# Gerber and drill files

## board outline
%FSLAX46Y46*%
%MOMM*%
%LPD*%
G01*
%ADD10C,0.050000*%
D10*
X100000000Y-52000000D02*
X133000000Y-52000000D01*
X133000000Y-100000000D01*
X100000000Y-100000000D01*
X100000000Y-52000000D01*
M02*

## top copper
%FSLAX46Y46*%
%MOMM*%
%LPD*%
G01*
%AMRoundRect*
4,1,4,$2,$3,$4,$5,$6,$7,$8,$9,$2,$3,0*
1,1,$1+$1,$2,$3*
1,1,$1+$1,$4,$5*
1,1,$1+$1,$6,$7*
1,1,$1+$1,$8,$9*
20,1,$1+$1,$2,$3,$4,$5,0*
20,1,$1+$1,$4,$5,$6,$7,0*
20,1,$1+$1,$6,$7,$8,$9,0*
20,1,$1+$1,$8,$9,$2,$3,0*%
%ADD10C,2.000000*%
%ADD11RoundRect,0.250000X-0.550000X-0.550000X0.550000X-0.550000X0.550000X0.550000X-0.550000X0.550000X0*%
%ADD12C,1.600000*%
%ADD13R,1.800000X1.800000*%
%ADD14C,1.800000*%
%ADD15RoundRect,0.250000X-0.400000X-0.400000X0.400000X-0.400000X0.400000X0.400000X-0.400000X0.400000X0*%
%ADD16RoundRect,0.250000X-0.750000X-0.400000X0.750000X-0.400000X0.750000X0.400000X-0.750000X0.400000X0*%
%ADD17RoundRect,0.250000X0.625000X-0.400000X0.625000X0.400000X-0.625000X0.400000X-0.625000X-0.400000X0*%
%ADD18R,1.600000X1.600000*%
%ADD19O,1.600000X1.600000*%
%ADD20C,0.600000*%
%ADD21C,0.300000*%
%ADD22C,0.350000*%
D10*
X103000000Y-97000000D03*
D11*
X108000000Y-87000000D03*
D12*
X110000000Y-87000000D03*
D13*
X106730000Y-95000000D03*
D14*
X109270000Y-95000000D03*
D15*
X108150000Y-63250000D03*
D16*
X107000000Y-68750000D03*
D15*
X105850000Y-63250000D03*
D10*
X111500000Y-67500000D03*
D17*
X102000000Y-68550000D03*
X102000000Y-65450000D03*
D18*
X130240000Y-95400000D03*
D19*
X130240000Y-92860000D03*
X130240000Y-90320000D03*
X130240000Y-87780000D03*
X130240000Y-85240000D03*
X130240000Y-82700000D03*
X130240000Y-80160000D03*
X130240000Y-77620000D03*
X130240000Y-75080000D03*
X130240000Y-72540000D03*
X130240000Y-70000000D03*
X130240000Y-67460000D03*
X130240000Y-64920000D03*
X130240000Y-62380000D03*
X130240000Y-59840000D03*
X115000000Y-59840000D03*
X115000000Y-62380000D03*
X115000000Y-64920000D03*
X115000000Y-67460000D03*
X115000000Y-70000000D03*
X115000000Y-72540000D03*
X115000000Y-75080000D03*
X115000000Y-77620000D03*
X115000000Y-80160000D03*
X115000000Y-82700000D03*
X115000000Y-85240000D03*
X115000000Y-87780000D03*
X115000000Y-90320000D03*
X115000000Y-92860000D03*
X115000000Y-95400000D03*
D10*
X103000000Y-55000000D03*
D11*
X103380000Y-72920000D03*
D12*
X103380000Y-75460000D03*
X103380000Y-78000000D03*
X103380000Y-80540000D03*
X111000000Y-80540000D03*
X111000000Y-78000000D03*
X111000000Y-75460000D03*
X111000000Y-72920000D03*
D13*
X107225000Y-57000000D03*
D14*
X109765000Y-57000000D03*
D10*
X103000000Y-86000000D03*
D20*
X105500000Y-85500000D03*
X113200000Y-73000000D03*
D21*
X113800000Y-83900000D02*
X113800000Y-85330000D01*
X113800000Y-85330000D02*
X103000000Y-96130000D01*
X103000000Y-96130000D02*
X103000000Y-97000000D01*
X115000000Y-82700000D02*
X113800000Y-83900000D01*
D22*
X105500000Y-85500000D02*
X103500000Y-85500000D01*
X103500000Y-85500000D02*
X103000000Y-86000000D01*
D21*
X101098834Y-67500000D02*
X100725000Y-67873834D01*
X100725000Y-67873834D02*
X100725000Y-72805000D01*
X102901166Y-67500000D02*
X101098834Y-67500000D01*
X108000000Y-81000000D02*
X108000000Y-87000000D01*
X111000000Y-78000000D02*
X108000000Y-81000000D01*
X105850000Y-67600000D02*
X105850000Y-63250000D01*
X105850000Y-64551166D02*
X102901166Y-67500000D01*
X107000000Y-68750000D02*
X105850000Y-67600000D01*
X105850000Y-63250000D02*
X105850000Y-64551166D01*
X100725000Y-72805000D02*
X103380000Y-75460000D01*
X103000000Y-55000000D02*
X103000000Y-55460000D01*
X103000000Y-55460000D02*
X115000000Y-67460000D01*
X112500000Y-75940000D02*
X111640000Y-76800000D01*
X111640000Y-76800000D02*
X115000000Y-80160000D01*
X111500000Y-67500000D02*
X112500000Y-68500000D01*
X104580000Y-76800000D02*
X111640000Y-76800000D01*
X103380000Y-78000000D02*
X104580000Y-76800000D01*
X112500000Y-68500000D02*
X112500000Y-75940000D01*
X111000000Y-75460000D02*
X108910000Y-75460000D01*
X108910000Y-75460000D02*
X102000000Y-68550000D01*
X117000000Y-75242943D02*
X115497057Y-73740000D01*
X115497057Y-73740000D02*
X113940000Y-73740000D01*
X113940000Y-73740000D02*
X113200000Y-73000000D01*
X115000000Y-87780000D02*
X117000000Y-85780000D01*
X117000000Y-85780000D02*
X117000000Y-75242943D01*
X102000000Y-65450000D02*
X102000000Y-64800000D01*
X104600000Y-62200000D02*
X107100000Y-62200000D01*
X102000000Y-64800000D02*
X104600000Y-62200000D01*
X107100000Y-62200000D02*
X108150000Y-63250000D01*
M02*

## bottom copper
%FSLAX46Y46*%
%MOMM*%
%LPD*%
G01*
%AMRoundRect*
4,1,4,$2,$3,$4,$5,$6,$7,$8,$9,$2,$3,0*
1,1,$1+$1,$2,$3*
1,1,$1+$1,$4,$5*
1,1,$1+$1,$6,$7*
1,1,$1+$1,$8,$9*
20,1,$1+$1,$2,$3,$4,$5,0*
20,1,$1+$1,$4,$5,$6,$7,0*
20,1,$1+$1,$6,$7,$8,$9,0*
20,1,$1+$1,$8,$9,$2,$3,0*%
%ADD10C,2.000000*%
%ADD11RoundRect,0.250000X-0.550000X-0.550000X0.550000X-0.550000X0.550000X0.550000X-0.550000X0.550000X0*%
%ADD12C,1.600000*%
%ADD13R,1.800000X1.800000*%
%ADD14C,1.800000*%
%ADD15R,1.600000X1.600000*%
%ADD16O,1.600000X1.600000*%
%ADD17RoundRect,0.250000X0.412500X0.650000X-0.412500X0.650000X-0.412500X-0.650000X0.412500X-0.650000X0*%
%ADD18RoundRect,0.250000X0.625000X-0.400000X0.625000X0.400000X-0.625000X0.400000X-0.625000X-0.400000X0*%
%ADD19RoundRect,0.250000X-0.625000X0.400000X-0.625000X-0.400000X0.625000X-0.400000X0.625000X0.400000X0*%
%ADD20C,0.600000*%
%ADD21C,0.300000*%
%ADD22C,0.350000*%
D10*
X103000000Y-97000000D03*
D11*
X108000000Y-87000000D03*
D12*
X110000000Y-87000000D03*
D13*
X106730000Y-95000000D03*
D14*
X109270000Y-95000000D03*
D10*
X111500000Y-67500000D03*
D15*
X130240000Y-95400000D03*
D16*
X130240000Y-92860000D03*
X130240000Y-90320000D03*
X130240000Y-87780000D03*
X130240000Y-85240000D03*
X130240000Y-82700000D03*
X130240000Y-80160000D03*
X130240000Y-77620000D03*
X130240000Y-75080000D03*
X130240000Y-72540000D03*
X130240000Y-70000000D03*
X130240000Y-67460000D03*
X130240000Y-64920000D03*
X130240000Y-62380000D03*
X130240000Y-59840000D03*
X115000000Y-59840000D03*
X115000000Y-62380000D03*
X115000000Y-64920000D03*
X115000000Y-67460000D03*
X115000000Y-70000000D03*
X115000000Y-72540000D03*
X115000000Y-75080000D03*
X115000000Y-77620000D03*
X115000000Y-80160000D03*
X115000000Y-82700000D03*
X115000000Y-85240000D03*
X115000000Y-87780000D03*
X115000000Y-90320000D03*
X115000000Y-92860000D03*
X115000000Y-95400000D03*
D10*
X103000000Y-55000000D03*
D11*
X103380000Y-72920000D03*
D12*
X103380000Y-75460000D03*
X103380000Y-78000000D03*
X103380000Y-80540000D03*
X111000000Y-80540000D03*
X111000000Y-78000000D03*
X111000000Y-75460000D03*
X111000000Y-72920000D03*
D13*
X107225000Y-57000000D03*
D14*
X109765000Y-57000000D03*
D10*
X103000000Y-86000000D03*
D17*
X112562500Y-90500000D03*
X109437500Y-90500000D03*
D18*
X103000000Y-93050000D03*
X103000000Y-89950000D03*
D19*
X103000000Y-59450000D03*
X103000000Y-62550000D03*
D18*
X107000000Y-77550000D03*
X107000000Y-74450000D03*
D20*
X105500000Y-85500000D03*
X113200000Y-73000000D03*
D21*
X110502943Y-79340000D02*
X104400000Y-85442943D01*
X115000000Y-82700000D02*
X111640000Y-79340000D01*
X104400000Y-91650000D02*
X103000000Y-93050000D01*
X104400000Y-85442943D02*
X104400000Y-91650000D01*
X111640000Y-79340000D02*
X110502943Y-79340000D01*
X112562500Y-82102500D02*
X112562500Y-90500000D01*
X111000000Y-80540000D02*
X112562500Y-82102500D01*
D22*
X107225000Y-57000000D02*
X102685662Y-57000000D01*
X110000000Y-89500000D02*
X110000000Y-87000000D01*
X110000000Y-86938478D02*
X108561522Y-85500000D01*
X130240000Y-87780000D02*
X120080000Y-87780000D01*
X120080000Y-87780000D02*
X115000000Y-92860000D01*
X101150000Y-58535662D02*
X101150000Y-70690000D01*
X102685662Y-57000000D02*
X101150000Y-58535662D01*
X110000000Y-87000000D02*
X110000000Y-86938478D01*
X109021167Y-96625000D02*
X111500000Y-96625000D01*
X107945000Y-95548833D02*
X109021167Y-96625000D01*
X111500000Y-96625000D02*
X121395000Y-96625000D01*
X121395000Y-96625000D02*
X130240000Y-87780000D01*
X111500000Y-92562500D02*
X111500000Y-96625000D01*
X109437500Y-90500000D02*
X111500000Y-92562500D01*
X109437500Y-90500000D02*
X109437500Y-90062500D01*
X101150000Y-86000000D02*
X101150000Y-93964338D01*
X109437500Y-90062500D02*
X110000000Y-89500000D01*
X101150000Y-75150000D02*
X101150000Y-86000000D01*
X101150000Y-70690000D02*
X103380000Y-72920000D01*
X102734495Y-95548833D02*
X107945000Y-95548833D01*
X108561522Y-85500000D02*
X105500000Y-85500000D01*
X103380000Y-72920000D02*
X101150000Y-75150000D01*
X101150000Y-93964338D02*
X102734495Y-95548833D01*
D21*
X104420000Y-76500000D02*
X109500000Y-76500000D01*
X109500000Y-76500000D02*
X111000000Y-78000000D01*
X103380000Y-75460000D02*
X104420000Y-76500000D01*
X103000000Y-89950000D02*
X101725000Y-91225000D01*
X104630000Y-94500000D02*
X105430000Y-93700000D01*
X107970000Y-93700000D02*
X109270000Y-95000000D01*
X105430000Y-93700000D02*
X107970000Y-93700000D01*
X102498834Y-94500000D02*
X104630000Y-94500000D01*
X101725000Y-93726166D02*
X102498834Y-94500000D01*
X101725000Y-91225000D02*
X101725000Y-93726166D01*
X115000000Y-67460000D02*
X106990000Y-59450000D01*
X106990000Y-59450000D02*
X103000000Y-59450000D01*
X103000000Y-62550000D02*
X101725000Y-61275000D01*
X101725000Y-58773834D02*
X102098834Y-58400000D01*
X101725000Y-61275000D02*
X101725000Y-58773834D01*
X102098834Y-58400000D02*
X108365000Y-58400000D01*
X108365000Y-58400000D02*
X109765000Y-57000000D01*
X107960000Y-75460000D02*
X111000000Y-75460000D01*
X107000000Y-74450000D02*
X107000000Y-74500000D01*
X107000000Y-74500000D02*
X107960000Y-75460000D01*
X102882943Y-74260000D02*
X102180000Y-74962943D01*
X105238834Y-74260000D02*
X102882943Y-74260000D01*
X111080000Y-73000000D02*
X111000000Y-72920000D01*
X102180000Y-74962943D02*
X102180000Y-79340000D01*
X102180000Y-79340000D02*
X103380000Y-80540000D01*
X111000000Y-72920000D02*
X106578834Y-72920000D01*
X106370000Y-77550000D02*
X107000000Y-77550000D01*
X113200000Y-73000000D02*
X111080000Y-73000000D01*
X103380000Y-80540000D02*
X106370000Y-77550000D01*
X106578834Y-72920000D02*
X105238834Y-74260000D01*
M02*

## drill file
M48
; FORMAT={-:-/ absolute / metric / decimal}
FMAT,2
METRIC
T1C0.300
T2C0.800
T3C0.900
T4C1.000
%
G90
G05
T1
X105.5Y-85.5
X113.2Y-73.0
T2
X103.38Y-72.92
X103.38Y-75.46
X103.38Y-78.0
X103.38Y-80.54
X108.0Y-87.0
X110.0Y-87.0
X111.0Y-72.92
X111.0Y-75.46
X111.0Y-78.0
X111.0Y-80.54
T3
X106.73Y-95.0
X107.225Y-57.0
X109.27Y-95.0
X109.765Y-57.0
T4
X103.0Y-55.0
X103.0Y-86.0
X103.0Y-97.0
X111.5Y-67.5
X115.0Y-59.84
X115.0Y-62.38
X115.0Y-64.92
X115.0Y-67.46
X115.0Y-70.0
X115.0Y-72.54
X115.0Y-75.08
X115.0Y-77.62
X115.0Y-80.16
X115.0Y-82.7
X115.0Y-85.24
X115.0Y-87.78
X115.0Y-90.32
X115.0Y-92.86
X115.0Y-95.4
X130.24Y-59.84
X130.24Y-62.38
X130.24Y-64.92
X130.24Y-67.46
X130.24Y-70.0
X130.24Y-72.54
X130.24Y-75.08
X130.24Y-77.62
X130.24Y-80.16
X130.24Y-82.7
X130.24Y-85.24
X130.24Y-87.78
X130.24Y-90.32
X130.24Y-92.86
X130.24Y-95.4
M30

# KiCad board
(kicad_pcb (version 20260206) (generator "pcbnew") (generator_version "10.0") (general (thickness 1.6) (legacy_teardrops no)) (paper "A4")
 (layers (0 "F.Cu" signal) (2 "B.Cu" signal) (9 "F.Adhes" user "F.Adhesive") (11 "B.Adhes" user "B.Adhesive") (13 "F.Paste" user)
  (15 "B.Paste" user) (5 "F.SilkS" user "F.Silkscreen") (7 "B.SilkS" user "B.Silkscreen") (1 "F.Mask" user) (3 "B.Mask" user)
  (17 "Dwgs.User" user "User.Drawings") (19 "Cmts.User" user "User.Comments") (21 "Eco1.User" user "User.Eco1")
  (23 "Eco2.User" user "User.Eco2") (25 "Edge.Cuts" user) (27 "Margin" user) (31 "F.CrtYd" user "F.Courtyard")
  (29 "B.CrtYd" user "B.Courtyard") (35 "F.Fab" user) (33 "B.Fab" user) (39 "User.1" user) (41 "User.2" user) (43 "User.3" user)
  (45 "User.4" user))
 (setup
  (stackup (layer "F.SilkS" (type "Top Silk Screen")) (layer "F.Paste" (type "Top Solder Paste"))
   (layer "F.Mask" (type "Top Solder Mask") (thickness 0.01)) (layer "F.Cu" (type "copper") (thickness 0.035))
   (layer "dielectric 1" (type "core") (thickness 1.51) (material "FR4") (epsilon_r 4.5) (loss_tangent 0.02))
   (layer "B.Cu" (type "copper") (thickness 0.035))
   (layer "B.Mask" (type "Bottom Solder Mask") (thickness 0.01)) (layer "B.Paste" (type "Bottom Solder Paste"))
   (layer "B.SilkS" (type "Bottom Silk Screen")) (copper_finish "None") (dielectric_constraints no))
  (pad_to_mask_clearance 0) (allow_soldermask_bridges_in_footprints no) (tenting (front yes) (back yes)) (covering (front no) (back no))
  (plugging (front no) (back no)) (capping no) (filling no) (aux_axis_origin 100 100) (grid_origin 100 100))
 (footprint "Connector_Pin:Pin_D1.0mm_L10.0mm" (layer "F.Cu") (at 103 97)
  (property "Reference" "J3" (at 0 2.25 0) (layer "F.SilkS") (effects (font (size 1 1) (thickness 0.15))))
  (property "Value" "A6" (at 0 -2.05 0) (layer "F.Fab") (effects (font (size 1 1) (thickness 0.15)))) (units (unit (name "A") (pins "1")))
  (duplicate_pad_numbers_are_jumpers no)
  (pad "1" thru_hole circle (at 0 0) (size 2 2) (drill 1) (layers "*.Cu" "*.Mask") (remove_unused_layers no) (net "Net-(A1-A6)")))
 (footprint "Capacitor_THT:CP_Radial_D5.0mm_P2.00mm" (layer "F.Cu") (at 108 87)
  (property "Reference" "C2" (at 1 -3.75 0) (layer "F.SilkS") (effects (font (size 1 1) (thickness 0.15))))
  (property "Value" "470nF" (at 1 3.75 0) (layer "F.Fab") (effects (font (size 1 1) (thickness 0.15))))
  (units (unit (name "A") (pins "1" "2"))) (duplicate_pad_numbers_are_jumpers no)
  (pad "1" thru_hole roundrect (at 0 0) (size 1.6 1.6) (drill 0.8) (layers "*.Cu" "*.Mask") (remove_unused_layers no)
   (roundrect_rratio 0.15625) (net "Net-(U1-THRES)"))
  (pad "2" thru_hole circle (at 2 0) (size 1.6 1.6) (drill 0.8) (layers "*.Cu" "*.Mask") (remove_unused_layers no) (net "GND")))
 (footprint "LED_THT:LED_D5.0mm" (layer "F.Cu") (at 106.73 95)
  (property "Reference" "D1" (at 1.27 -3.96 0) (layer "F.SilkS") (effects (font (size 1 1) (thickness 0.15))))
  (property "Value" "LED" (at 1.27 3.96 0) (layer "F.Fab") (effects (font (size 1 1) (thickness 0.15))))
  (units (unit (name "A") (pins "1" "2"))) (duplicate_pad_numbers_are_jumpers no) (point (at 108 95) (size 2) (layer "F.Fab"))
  (pad "1" thru_hole rect (at 0 0) (size 1.8 1.8) (drill 0.9) (layers "*.Cu" "*.Mask") (remove_unused_layers no) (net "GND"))
  (pad "2" thru_hole circle (at 2.54 0) (size 1.8 1.8) (drill 0.9) (layers "*.Cu" "*.Mask") (remove_unused_layers no) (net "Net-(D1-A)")))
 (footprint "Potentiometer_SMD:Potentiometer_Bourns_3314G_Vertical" (layer "F.Cu") (at 107 66)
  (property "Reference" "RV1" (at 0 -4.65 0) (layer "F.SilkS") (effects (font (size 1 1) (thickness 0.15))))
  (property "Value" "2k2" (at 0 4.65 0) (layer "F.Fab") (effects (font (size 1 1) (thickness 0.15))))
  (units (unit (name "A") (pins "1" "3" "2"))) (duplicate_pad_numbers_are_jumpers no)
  (pad "1" smd roundrect (at 1.15 -2.75) (size 1.3 1.3) (layers "F.Cu" "F.Mask" "F.Paste") (roundrect_rratio 0.192308) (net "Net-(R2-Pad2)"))
  (pad "2" smd roundrect (at 0 2.75) (size 2 1.3) (layers "F.Cu" "F.Mask" "F.Paste") (roundrect_rratio 0.192308) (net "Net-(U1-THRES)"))
  (pad "3" smd roundrect (at -1.15 -2.75) (size 1.3 1.3) (layers "F.Cu" "F.Mask" "F.Paste") (roundrect_rratio 0.192308)
   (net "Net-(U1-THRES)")))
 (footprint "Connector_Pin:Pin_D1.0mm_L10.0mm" (layer "F.Cu") (at 111.5 67.5)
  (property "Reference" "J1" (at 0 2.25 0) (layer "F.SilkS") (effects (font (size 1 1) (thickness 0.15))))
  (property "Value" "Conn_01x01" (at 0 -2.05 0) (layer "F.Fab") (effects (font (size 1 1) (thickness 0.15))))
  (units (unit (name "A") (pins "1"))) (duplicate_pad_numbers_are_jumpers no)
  (pad "1" thru_hole circle (at 0 0) (size 2 2) (drill 1) (layers "*.Cu" "*.Mask") (remove_unused_layers no) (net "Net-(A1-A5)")))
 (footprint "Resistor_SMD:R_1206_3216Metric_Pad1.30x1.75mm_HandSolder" (layer "F.Cu") (at 102 67 90)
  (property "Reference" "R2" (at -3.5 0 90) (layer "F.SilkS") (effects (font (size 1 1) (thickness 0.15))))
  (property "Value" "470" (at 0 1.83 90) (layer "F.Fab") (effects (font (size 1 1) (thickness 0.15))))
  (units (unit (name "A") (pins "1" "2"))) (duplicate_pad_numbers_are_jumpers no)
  (pad "1" smd roundrect (at -1.55 0 90) (size 1.3 1.75) (layers "F.Cu" "F.Mask" "F.Paste") (roundrect_rratio 0.192308)
   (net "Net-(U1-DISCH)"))
  (pad "2" smd roundrect (at 1.55 0 90) (size 1.3 1.75) (layers "F.Cu" "F.Mask" "F.Paste") (roundrect_rratio 0.192308) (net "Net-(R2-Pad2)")))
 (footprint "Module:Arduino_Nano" (layer "F.Cu") (at 130.24 95.4 180)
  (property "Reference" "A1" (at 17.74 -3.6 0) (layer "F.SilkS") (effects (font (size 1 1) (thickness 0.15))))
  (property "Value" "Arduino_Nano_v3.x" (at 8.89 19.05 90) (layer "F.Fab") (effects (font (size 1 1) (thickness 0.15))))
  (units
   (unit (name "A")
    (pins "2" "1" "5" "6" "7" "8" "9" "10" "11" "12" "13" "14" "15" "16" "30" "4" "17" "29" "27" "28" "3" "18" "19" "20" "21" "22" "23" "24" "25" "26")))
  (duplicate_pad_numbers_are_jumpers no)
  (pad "1" thru_hole rect (at 0 0 180) (size 1.6 1.6) (drill 1) (layers "*.Cu" "*.Mask") (remove_unused_layers no)
   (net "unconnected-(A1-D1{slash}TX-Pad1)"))
  (pad "2" thru_hole oval (at 0 2.54 180) (size 1.6 1.6) (drill 1) (layers "*.Cu" "*.Mask") (remove_unused_layers no)
   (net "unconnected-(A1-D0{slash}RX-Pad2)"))
  (pad "3" thru_hole oval (at 0 5.08 180) (size 1.6 1.6) (drill 1) (layers "*.Cu" "*.Mask") (remove_unused_layers no)
   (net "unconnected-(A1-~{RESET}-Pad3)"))
  (pad "4" thru_hole oval (at 0 7.62 180) (size 1.6 1.6) (drill 1) (layers "*.Cu" "*.Mask") (remove_unused_layers no) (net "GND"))
  (pad "5" thru_hole oval (at 0 10.16 180) (size 1.6 1.6) (drill 1) (layers "*.Cu" "*.Mask") (remove_unused_layers no)
   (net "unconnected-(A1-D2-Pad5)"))
  (pad "6" thru_hole oval (at 0 12.7 180) (size 1.6 1.6) (drill 1) (layers "*.Cu" "*.Mask") (remove_unused_layers no)
   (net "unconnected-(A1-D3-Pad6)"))
  (pad "7" thru_hole oval (at 0 15.24 180) (size 1.6 1.6) (drill 1) (layers "*.Cu" "*.Mask") (remove_unused_layers no)
   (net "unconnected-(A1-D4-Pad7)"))
  (pad "8" thru_hole oval (at 0 17.78 180) (size 1.6 1.6) (drill 1) (layers "*.Cu" "*.Mask") (remove_unused_layers no)
   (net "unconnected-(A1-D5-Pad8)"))
  (pad "9" thru_hole oval (at 0 20.32 180) (size 1.6 1.6) (drill 1) (layers "*.Cu" "*.Mask") (remove_unused_layers no)
   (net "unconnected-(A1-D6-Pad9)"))
  (pad "10" thru_hole oval (at 0 22.86 180) (size 1.6 1.6) (drill 1) (layers "*.Cu" "*.Mask") (remove_unused_layers no)
   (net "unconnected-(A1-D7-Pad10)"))
  (pad "11" thru_hole oval (at 0 25.4 180) (size 1.6 1.6) (drill 1) (layers "*.Cu" "*.Mask") (remove_unused_layers no)
   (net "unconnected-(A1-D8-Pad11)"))
  (pad "12" thru_hole oval (at 0 27.94 180) (size 1.6 1.6) (drill 1) (layers "*.Cu" "*.Mask") (remove_unused_layers no)
   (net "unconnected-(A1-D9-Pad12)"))
  (pad "13" thru_hole oval (at 0 30.48 180) (size 1.6 1.6) (drill 1) (layers "*.Cu" "*.Mask") (remove_unused_layers no)
   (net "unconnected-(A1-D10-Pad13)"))
  (pad "14" thru_hole oval (at 0 33.02 180) (size 1.6 1.6) (drill 1) (layers "*.Cu" "*.Mask") (remove_unused_layers no)
   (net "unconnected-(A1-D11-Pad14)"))
  (pad "15" thru_hole oval (at 0 35.56 180) (size 1.6 1.6) (drill 1) (layers "*.Cu" "*.Mask") (remove_unused_layers no)
   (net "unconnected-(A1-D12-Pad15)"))
  (pad "16" thru_hole oval (at 15.24 35.56 180) (size 1.6 1.6) (drill 1) (layers "*.Cu" "*.Mask") (remove_unused_layers no)
   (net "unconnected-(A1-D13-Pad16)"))
  (pad "17" thru_hole oval (at 15.24 33.02 180) (size 1.6 1.6) (drill 1) (layers "*.Cu" "*.Mask") (remove_unused_layers no)
   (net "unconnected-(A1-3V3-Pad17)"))
  (pad "18" thru_hole oval (at 15.24 30.48 180) (size 1.6 1.6) (drill 1) (layers "*.Cu" "*.Mask") (remove_unused_layers no)
   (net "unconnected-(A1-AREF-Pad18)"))
  (pad "19" thru_hole oval (at 15.24 27.94 180) (size 1.6 1.6) (drill 1) (layers "*.Cu" "*.Mask") (remove_unused_layers no)
   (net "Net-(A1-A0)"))
  (pad "20" thru_hole oval (at 15.24 25.4 180) (size 1.6 1.6) (drill 1) (layers "*.Cu" "*.Mask") (remove_unused_layers no)
   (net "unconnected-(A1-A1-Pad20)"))
  (pad "21" thru_hole oval (at 15.24 22.86 180) (size 1.6 1.6) (drill 1) (layers "*.Cu" "*.Mask") (remove_unused_layers no)
   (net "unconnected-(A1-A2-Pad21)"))
  (pad "22" thru_hole oval (at 15.24 20.32 180) (size 1.6 1.6) (drill 1) (layers "*.Cu" "*.Mask") (remove_unused_layers no)
   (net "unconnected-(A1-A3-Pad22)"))
  (pad "23" thru_hole oval (at 15.24 17.78 180) (size 1.6 1.6) (drill 1) (layers "*.Cu" "*.Mask") (remove_unused_layers no)
   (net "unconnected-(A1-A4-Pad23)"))
  (pad "24" thru_hole oval (at 15.24 15.24 180) (size 1.6 1.6) (drill 1) (layers "*.Cu" "*.Mask") (remove_unused_layers no)
   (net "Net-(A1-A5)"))
  (pad "25" thru_hole oval (at 15.24 12.7 180) (size 1.6 1.6) (drill 1) (layers "*.Cu" "*.Mask") (remove_unused_layers no)
   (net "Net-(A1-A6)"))
  (pad "26" thru_hole oval (at 15.24 10.16 180) (size 1.6 1.6) (drill 1) (layers "*.Cu" "*.Mask") (remove_unused_layers no)
   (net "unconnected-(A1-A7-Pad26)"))
  (pad "27" thru_hole oval (at 15.24 7.62 180) (size 1.6 1.6) (drill 1) (layers "*.Cu" "*.Mask") (remove_unused_layers no) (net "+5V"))
  (pad "28" thru_hole oval (at 15.24 5.08 180) (size 1.6 1.6) (drill 1) (layers "*.Cu" "*.Mask") (remove_unused_layers no)
   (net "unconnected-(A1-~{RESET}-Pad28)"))
  (pad "29" thru_hole oval (at 15.24 2.54 180) (size 1.6 1.6) (drill 1) (layers "*.Cu" "*.Mask") (remove_unused_layers no) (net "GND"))
  (pad "30" thru_hole oval (at 15.24 0 180) (size 1.6 1.6) (drill 1) (layers "*.Cu" "*.Mask") (remove_unused_layers no)
   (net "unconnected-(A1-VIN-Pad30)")))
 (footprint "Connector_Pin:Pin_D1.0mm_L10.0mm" (layer "F.Cu") (at 103 55)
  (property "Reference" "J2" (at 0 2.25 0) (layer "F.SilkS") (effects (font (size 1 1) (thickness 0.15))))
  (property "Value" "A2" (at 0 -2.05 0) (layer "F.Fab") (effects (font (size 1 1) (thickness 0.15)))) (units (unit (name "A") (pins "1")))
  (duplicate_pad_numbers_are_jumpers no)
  (pad "1" thru_hole circle (at 0 0) (size 2 2) (drill 1) (layers "*.Cu" "*.Mask") (remove_unused_layers no) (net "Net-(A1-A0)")))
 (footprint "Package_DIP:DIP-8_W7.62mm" (layer "F.Cu") (at 103.38 72.92)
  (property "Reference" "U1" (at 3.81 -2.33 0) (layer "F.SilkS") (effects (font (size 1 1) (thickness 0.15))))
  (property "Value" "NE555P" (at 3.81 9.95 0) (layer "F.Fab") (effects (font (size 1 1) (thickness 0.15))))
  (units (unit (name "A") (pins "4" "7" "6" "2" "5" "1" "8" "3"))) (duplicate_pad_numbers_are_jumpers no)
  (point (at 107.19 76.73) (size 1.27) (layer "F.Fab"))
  (pad "1" thru_hole roundrect (at 0 0) (size 1.6 1.6) (drill 0.8) (layers "*.Cu" "*.Mask") (remove_unused_layers no)
   (roundrect_rratio 0.15625) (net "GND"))
  (pad "2" thru_hole circle (at 0 2.54) (size 1.6 1.6) (drill 0.8) (layers "*.Cu" "*.Mask") (remove_unused_layers no) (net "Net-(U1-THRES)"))
  (pad "3" thru_hole circle (at 0 5.08) (size 1.6 1.6) (drill 0.8) (layers "*.Cu" "*.Mask") (remove_unused_layers no) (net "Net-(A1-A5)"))
  (pad "4" thru_hole circle (at 0 7.62) (size 1.6 1.6) (drill 0.8) (layers "*.Cu" "*.Mask") (remove_unused_layers no) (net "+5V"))
  (pad "5" thru_hole circle (at 7.62 7.62) (size 1.6 1.6) (drill 0.8) (layers "*.Cu" "*.Mask") (remove_unused_layers no)
   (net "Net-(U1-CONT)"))
  (pad "6" thru_hole circle (at 7.62 5.08) (size 1.6 1.6) (drill 0.8) (layers "*.Cu" "*.Mask") (remove_unused_layers no)
   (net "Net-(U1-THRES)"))
  (pad "7" thru_hole circle (at 7.62 2.54) (size 1.6 1.6) (drill 0.8) (layers "*.Cu" "*.Mask") (remove_unused_layers no)
   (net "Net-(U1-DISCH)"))
  (pad "8" thru_hole circle (at 7.62 0) (size 1.6 1.6) (drill 0.8) (layers "*.Cu" "*.Mask") (remove_unused_layers no) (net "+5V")))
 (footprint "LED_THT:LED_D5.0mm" (layer "F.Cu") (at 107.225 57)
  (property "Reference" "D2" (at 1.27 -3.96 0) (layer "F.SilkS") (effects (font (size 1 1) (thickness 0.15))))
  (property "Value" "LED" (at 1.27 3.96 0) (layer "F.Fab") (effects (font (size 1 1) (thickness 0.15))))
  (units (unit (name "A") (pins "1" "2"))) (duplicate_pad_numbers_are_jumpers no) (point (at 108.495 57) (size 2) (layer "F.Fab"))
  (pad "1" thru_hole rect (at 0 0) (size 1.8 1.8) (drill 0.9) (layers "*.Cu" "*.Mask") (remove_unused_layers no) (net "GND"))
  (pad "2" thru_hole circle (at 2.54 0) (size 1.8 1.8) (drill 0.9) (layers "*.Cu" "*.Mask") (remove_unused_layers no) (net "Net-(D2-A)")))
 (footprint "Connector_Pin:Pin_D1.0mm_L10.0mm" (layer "F.Cu") (at 103 86)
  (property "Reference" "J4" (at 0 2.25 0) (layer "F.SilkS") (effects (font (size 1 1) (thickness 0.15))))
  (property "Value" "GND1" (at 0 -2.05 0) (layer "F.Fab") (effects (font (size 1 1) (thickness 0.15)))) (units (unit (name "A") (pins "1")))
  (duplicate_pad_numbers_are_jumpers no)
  (pad "1" thru_hole circle (at 0 0) (size 2 2) (drill 1) (layers "*.Cu" "*.Mask") (remove_unused_layers no) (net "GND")))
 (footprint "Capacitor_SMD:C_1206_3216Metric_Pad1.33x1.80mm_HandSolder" (layer "B.Cu") (at 111 90.5 180)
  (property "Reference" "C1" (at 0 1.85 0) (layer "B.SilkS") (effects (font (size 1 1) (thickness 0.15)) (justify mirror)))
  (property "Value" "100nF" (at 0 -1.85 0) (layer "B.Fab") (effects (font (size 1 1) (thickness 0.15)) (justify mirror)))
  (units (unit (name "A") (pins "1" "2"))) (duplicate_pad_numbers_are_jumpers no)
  (pad "1" smd roundrect (at -1.5625 0 180) (size 1.325 1.8) (layers "B.Cu" "B.Mask" "B.Paste") (roundrect_rratio 0.188679)
   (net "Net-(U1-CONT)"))
  (pad "2" smd roundrect (at 1.5625 0 180) (size 1.325 1.8) (layers "B.Cu" "B.Mask" "B.Paste") (roundrect_rratio 0.188679) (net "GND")))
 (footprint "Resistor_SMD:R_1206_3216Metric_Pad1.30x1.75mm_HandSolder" (layer "B.Cu") (at 103 91.5 90)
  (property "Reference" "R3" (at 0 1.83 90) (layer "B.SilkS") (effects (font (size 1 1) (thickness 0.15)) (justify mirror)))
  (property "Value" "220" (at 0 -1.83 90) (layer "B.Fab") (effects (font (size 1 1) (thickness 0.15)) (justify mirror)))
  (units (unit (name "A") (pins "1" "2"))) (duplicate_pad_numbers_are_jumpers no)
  (pad "1" smd roundrect (at -1.55 0 90) (size 1.3 1.75) (layers "B.Cu" "B.Mask" "B.Paste") (roundrect_rratio 0.192308) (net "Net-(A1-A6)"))
  (pad "2" smd roundrect (at 1.55 0 90) (size 1.3 1.75) (layers "B.Cu" "B.Mask" "B.Paste") (roundrect_rratio 0.192308) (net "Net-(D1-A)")))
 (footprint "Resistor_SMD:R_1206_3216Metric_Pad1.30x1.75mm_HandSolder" (layer "B.Cu") (at 103 61 -90)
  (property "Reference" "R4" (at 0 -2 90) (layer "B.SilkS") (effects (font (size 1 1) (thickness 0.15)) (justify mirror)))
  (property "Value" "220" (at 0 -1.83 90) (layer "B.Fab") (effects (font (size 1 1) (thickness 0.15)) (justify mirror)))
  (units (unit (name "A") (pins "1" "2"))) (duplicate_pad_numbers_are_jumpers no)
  (pad "1" smd roundrect (at -1.55 0 270) (size 1.3 1.75) (layers "B.Cu" "B.Mask" "B.Paste") (roundrect_rratio 0.192308) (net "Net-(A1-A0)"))
  (pad "2" smd roundrect (at 1.55 0 270) (size 1.3 1.75) (layers "B.Cu" "B.Mask" "B.Paste") (roundrect_rratio 0.192308) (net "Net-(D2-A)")))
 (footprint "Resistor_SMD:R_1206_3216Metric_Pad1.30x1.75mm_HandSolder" (layer "B.Cu") (at 107 76 90)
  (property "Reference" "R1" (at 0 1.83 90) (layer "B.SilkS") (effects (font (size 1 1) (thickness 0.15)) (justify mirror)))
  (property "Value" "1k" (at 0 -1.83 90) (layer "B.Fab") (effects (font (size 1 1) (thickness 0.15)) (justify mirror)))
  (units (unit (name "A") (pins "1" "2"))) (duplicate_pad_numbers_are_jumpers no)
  (pad "1" smd roundrect (at -1.55 0 90) (size 1.3 1.75) (layers "B.Cu" "B.Mask" "B.Paste") (roundrect_rratio 0.192308) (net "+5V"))
  (pad "2" smd roundrect (at 1.55 0 90) (size 1.3 1.75) (layers "B.Cu" "B.Mask" "B.Paste") (roundrect_rratio 0.192308)
   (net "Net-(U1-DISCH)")))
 (gr_rect (start 100 52) (end 133 100) (stroke (width 0.05) (type solid)) (fill no) (layer "Edge.Cuts"))
 (segment (start 113.8 83.9) (end 113.8 85.33) (width 0.3) (layer "F.Cu") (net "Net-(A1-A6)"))
 (segment (start 113.8 85.33) (end 103 96.13) (width 0.3) (layer "F.Cu") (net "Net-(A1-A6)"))
 (segment (start 103 96.13) (end 103 97) (width 0.3) (layer "F.Cu") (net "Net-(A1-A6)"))
 (segment (start 115 82.7) (end 113.8 83.9) (width 0.3) (layer "F.Cu") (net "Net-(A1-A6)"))
 (segment (start 110.502943 79.34) (end 104.4 85.442943) (width 0.3) (layer "B.Cu") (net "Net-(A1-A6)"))
 (segment (start 115 82.7) (end 111.64 79.34) (width 0.3) (layer "B.Cu") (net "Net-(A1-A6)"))
 (segment (start 104.4 91.65) (end 103 93.05) (width 0.3) (layer "B.Cu") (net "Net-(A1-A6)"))
 (segment (start 104.4 85.442943) (end 104.4 91.65) (width 0.3) (layer "B.Cu") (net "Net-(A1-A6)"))
 (segment (start 111.64 79.34) (end 110.502943 79.34) (width 0.3) (layer "B.Cu") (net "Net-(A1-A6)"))
 (segment (start 112.5625 82.1025) (end 112.5625 90.5) (width 0.3) (layer "B.Cu") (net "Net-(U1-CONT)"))
 (segment (start 111 80.54) (end 112.5625 82.1025) (width 0.3) (layer "B.Cu") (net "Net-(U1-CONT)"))
 (segment (start 105.5 85.5) (end 103.5 85.5) (width 0.35) (layer "F.Cu") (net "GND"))
 (segment (start 103.5 85.5) (end 103 86) (width 0.35) (layer "F.Cu") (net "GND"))
 (via (at 105.5 85.5) (size 0.6) (drill 0.3) (layers "F.Cu" "B.Cu") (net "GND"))
 (segment (start 107.225 57) (end 102.685662 57) (width 0.35) (layer "B.Cu") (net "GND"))
 (segment (start 110 89.5) (end 110 87) (width 0.35) (layer "B.Cu") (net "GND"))
 (segment (start 110 86.938478) (end 108.561522 85.5) (width 0.35) (layer "B.Cu") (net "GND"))
 (segment (start 130.24 87.78) (end 120.08 87.78) (width 0.35) (layer "B.Cu") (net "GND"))
 (segment (start 120.08 87.78) (end 115 92.86) (width 0.35) (layer "B.Cu") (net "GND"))
 (segment (start 101.15 58.535662) (end 101.15 70.69) (width 0.35) (layer "B.Cu") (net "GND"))
 (segment (start 102.685662 57) (end 101.15 58.535662) (width 0.35) (layer "B.Cu") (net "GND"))
 (segment (start 110 87) (end 110 86.938478) (width 0.35) (layer "B.Cu") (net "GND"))
 (segment (start 109.021167 96.625) (end 111.5 96.625) (width 0.35) (layer "B.Cu") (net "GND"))
 (segment (start 107.945 95.548833) (end 109.021167 96.625) (width 0.35) (layer "B.Cu") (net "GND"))
 (segment (start 111.5 96.625) (end 121.395 96.625) (width 0.35) (layer "B.Cu") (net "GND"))
 (segment (start 121.395 96.625) (end 130.24 87.78) (width 0.35) (layer "B.Cu") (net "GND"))
 (segment (start 111.5 92.5625) (end 111.5 96.625) (width 0.35) (layer "B.Cu") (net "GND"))
 (segment (start 109.4375 90.5) (end 111.5 92.5625) (width 0.35) (layer "B.Cu") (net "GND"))
 (segment (start 109.4375 90.5) (end 109.4375 90.0625) (width 0.35) (layer "B.Cu") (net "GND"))
 (segment (start 101.15 86) (end 101.15 93.964338) (width 0.35) (layer "B.Cu") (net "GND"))
 (segment (start 109.4375 90.0625) (end 110 89.5) (width 0.35) (layer "B.Cu") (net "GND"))
 (segment (start 101.15 75.15) (end 101.15 86) (width 0.35) (layer "B.Cu") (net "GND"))
 (segment (start 101.15 70.69) (end 103.38 72.92) (width 0.35) (layer "B.Cu") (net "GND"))
 (segment (start 102.734495 95.548833) (end 107.945 95.548833) (width 0.35) (layer "B.Cu") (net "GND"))
 (segment (start 108.561522 85.5) (end 105.5 85.5) (width 0.35) (layer "B.Cu") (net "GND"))
 (segment (start 103.38 72.92) (end 101.15 75.15) (width 0.35) (layer "B.Cu") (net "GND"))
 (segment (start 101.15 93.964338) (end 102.734495 95.548833) (width 0.35) (layer "B.Cu") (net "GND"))
 (segment (start 101.098834 67.5) (end 100.725 67.873834) (width 0.3) (layer "F.Cu") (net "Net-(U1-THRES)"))
 (segment (start 100.725 67.873834) (end 100.725 72.805) (width 0.3) (layer "F.Cu") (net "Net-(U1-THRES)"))
 (segment (start 102.901166 67.5) (end 101.098834 67.5) (width 0.3) (layer "F.Cu") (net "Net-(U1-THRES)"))
 (segment (start 108 81) (end 108 87) (width 0.3) (layer "F.Cu") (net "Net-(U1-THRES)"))
 (segment (start 111 78) (end 108 81) (width 0.3) (layer "F.Cu") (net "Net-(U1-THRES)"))
 (segment (start 105.85 67.6) (end 105.85 63.25) (width 0.3) (layer "F.Cu") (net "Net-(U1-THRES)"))
 (segment (start 105.85 64.551166) (end 102.901166 67.5) (width 0.3) (layer "F.Cu") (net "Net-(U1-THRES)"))
 (segment (start 107 68.75) (end 105.85 67.6) (width 0.3) (layer "F.Cu") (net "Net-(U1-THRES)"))
 (segment (start 105.85 63.25) (end 105.85 64.551166) (width 0.3) (layer "F.Cu") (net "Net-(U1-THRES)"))
 (segment (start 100.725 72.805) (end 103.38 75.46) (width 0.3) (layer "F.Cu") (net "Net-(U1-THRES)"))
 (segment (start 104.42 76.5) (end 109.5 76.5) (width 0.3) (layer "B.Cu") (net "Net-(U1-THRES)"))
 (segment (start 109.5 76.5) (end 111 78) (width 0.3) (layer "B.Cu") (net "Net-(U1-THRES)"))
 (segment (start 103.38 75.46) (end 104.42 76.5) (width 0.3) (layer "B.Cu") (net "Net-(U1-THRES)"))
 (segment (start 103 89.95) (end 101.725 91.225) (width 0.3) (layer "B.Cu") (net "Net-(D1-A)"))
 (segment (start 104.63 94.5) (end 105.43 93.7) (width 0.3) (layer "B.Cu") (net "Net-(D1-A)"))
 (segment (start 107.97 93.7) (end 109.27 95) (width 0.3) (layer "B.Cu") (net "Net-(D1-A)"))
 (segment (start 105.43 93.7) (end 107.97 93.7) (width 0.3) (layer "B.Cu") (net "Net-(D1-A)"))
 (segment (start 102.498834 94.5) (end 104.63 94.5) (width 0.3) (layer "B.Cu") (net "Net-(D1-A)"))
 (segment (start 101.725 93.726166) (end 102.498834 94.5) (width 0.3) (layer "B.Cu") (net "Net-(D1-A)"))
 (segment (start 101.725 91.225) (end 101.725 93.726166) (width 0.3) (layer "B.Cu") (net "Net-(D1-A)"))
 (segment (start 103 55) (end 103 55.46) (width 0.3) (layer "F.Cu") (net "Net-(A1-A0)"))
 (segment (start 103 55.46) (end 115 67.46) (width 0.3) (layer "F.Cu") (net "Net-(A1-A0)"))
 (segment (start 115 67.46) (end 106.99 59.45) (width 0.3) (layer "B.Cu") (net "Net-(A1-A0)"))
 (segment (start 106.99 59.45) (end 103 59.45) (width 0.3) (layer "B.Cu") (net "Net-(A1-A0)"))
 (segment (start 103 62.55) (end 101.725 61.275) (width 0.3) (layer "B.Cu") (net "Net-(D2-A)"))
 (segment (start 101.725 58.773834) (end 102.098834 58.4) (width 0.3) (layer "B.Cu") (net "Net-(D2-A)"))
 (segment (start 101.725 61.275) (end 101.725 58.773834) (width 0.3) (layer "B.Cu") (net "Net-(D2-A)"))
 (segment (start 102.098834 58.4) (end 108.365 58.4) (width 0.3) (layer "B.Cu") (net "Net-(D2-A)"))
 (segment (start 108.365 58.4) (end 109.765 57) (width 0.3) (layer "B.Cu") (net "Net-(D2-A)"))
 (segment (start 112.5 75.94) (end 111.64 76.8) (width 0.3) (layer "F.Cu") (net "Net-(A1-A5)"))
 (segment (start 111.64 76.8) (end 115 80.16) (width 0.3) (layer "F.Cu") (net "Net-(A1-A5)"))
 (segment (start 111.5 67.5) (end 112.5 68.5) (width 0.3) (layer "F.Cu") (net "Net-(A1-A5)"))
 (segment (start 104.58 76.8) (end 111.64 76.8) (width 0.3) (layer "F.Cu") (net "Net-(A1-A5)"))
 (segment (start 103.38 78) (end 104.58 76.8) (width 0.3) (layer "F.Cu") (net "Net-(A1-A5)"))
 (segment (start 112.5 68.5) (end 112.5 75.94) (width 0.3) (layer "F.Cu") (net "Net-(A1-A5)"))
 (segment (start 111 75.46) (end 108.91 75.46) (width 0.3) (layer "F.Cu") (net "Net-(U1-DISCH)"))
 (segment (start 108.91 75.46) (end 102 68.55) (width 0.3) (layer "F.Cu") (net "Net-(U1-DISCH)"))
 (segment (start 107.96 75.46) (end 111 75.46) (width 0.3) (layer "B.Cu") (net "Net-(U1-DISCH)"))
 (segment (start 107 74.45) (end 107 74.5) (width 0.3) (layer "B.Cu") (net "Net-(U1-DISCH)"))
 (segment (start 107 74.5) (end 107.96 75.46) (width 0.3) (layer "B.Cu") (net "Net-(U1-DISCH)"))
 (segment (start 117 75.242943) (end 115.497057 73.74) (width 0.3) (layer "F.Cu") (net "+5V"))
 (segment (start 115.497057 73.74) (end 113.94 73.74) (width 0.3) (layer "F.Cu") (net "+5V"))
 (segment (start 113.94 73.74) (end 113.2 73) (width 0.3) (layer "F.Cu") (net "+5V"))
 (segment (start 115 87.78) (end 117 85.78) (width 0.3) (layer "F.Cu") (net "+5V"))
 (segment (start 117 85.78) (end 117 75.242943) (width 0.3) (layer "F.Cu") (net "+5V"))
 (via (at 113.2 73) (size 0.6) (drill 0.3) (layers "F.Cu" "B.Cu") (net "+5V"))
 (segment (start 102.882943 74.26) (end 102.18 74.962943) (width 0.3) (layer "B.Cu") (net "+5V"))
 (segment (start 105.238834 74.26) (end 102.882943 74.26) (width 0.3) (layer "B.Cu") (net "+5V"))
 (segment (start 111.08 73) (end 111 72.92) (width 0.3) (layer "B.Cu") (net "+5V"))
 (segment (start 102.18 74.962943) (end 102.18 79.34) (width 0.3) (layer "B.Cu") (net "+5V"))
 (segment (start 102.18 79.34) (end 103.38 80.54) (width 0.3) (layer "B.Cu") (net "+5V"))
 (segment (start 111 72.92) (end 106.578834 72.92) (width 0.3) (layer "B.Cu") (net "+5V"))
 (segment (start 106.37 77.55) (end 107 77.55) (width 0.3) (layer "B.Cu") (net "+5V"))
 (segment (start 113.2 73) (end 111.08 73) (width 0.3) (layer "B.Cu") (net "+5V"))
 (segment (start 103.38 80.54) (end 106.37 77.55) (width 0.3) (layer "B.Cu") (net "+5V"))
 (segment (start 106.578834 72.92) (end 105.238834 74.26) (width 0.3) (layer "B.Cu") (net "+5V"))
 (segment (start 102 65.45) (end 102 64.8) (width 0.3) (layer "F.Cu") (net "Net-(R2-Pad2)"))
 (segment (start 104.6 62.2) (end 107.1 62.2) (width 0.3) (layer "F.Cu") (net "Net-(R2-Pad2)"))
 (segment (start 102 64.8) (end 104.6 62.2) (width 0.3) (layer "F.Cu") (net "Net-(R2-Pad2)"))
 (segment (start 107.1 62.2) (end 108.15 63.25) (width 0.3) (layer "F.Cu") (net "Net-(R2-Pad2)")))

